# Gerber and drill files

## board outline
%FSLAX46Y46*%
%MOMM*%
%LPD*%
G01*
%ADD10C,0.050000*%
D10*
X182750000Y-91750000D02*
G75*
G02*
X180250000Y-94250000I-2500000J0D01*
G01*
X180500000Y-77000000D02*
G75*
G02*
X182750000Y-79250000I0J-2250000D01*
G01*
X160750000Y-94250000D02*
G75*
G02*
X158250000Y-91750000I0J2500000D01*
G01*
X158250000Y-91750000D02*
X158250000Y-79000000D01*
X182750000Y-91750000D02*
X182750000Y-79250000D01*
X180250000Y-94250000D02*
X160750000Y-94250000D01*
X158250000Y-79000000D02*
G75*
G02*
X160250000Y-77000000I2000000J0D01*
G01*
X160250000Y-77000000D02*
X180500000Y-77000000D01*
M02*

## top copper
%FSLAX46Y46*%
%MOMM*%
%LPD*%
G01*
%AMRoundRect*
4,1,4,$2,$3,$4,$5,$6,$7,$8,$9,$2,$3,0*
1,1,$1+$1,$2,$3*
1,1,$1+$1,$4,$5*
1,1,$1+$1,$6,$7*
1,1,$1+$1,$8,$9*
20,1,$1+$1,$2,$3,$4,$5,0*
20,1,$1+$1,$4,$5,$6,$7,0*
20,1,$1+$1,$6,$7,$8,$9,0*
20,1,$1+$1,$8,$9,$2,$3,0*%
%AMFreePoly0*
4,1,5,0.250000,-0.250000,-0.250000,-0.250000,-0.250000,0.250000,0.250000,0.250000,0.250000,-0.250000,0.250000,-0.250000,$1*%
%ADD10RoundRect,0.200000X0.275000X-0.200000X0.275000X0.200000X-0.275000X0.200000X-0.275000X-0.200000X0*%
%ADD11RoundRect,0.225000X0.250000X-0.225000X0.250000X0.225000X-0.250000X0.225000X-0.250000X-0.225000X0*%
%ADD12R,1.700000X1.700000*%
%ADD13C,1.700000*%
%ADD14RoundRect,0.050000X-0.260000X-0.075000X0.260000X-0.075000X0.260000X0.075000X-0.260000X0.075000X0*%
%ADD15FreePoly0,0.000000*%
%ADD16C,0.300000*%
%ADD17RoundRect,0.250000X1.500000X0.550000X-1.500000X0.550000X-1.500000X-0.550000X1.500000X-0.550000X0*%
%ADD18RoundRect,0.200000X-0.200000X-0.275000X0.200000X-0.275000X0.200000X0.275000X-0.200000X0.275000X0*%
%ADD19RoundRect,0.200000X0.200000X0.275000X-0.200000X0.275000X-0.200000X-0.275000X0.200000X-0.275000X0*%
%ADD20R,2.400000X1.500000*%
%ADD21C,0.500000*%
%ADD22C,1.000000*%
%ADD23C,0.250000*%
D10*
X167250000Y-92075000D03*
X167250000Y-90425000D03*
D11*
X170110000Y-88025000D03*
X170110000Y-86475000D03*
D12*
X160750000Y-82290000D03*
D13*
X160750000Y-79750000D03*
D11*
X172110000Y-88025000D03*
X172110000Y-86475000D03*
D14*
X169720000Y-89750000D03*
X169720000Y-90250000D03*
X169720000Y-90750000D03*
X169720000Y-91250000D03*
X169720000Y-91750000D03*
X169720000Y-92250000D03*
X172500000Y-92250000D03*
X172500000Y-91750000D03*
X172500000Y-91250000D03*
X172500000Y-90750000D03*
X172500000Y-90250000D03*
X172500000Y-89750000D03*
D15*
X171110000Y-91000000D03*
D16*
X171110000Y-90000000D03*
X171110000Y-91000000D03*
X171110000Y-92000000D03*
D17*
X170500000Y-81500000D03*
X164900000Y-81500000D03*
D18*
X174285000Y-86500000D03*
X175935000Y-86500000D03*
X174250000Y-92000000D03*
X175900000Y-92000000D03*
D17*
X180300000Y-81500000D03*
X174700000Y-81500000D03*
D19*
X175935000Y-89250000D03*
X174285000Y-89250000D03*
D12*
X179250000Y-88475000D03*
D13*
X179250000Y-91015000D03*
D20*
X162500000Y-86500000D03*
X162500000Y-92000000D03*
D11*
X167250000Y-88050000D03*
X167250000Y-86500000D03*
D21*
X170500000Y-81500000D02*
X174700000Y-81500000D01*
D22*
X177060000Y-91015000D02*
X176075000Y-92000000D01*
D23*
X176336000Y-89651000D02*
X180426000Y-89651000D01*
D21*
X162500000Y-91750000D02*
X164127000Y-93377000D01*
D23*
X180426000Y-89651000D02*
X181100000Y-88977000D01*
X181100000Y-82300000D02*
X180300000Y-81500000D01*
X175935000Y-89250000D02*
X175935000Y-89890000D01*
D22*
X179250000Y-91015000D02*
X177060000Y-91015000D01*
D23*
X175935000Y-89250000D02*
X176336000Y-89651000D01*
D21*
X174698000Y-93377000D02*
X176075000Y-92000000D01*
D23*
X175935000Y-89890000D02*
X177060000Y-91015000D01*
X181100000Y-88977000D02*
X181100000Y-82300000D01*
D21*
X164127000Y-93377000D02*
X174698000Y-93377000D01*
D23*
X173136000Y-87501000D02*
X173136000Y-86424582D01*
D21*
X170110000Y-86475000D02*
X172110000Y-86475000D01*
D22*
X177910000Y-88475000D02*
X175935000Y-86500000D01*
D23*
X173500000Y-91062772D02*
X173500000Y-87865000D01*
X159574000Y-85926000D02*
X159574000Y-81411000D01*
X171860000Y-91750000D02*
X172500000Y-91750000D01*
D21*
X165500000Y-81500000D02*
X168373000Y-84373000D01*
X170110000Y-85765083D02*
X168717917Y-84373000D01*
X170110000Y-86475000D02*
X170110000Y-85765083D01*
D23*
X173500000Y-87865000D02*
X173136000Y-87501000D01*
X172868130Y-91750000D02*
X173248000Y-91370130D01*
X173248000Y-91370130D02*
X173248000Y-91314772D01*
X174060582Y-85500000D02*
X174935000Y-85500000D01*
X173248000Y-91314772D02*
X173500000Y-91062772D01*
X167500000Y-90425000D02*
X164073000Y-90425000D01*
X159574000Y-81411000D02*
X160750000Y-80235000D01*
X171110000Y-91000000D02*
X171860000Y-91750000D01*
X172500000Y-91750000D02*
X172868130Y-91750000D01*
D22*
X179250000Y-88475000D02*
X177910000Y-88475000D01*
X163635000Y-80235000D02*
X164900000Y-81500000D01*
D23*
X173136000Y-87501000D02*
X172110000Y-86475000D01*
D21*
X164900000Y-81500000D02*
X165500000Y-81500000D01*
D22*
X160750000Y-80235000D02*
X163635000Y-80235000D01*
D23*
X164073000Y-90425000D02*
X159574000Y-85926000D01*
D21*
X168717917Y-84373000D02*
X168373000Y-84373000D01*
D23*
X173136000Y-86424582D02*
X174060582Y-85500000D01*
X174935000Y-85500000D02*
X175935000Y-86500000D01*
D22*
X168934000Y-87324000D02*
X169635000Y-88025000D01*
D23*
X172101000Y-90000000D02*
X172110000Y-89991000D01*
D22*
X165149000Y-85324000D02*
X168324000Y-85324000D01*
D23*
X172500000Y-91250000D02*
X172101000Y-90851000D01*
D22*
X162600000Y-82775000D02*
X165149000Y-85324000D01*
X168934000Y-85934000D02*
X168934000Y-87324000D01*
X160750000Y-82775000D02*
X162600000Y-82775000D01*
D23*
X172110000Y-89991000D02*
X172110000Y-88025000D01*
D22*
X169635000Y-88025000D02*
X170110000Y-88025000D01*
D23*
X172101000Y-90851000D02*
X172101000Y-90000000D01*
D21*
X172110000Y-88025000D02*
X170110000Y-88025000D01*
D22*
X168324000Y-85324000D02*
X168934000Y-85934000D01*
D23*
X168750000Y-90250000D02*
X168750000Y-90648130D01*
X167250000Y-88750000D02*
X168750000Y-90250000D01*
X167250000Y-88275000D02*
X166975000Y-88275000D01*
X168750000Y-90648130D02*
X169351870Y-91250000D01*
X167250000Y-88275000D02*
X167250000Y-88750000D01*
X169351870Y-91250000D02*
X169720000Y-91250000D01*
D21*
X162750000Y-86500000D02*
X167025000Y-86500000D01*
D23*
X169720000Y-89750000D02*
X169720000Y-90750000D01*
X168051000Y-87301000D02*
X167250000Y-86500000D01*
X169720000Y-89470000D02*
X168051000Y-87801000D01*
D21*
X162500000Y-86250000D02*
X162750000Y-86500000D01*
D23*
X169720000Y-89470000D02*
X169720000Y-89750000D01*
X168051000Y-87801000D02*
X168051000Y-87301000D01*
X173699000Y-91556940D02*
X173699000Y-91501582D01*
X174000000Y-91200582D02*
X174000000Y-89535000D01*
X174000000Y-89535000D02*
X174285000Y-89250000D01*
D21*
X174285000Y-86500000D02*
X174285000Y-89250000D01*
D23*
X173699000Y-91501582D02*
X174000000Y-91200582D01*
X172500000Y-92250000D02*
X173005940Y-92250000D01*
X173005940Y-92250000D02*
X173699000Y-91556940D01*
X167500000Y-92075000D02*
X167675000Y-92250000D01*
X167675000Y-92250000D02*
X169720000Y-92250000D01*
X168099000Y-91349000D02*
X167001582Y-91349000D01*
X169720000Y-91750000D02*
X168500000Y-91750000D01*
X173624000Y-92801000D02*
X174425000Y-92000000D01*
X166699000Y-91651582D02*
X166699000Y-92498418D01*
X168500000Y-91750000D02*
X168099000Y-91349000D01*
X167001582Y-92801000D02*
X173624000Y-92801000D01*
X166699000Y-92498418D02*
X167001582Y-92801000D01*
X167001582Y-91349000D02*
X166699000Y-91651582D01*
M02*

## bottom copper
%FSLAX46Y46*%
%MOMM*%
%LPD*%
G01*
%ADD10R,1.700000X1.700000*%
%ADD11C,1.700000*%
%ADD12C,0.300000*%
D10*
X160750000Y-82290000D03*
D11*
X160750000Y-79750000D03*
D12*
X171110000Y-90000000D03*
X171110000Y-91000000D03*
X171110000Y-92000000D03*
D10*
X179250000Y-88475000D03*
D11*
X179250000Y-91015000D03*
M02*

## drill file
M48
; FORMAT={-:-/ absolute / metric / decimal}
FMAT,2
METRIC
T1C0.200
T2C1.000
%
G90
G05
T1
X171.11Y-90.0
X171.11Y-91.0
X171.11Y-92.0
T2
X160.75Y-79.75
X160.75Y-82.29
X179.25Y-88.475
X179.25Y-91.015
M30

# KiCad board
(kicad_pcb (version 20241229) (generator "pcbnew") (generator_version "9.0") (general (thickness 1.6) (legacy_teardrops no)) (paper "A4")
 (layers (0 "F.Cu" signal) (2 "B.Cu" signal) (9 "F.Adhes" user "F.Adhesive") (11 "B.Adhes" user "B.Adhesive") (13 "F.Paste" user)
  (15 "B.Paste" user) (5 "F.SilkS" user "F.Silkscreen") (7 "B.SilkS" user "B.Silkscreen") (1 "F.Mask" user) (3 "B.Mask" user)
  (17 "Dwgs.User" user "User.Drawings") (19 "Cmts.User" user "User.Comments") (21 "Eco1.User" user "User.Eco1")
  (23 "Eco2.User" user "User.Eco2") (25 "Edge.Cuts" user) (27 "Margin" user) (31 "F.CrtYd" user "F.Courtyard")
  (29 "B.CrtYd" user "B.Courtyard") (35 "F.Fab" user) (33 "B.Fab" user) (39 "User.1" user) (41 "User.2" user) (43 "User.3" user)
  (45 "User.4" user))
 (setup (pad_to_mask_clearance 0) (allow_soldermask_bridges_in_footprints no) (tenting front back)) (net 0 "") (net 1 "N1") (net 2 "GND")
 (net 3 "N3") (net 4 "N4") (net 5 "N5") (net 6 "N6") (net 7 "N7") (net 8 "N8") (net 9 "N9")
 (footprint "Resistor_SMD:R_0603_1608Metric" (layer "F.Cu") (at 167.25 91.25 90)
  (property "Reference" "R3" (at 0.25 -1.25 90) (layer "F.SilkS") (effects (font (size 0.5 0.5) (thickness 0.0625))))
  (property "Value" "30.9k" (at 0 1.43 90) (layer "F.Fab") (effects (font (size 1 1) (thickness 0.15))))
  (pad "1" smd roundrect (at -0.825 0 90) (size 0.8 0.95) (layers "F.Cu" "F.Mask" "F.Paste") (roundrect_rratio 0.25) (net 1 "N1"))
  (pad "2" smd roundrect (at 0.825 0 90) (size 0.8 0.95) (layers "F.Cu" "F.Mask" "F.Paste") (roundrect_rratio 0.25) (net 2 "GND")))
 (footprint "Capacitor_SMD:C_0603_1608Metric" (layer "F.Cu") (at 170.11 87.25 90)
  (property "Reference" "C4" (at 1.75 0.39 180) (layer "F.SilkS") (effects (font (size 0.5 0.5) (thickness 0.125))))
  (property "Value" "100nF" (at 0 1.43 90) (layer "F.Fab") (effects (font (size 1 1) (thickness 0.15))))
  (pad "1" smd roundrect (at -0.775 0 90) (size 0.9 0.95) (layers "F.Cu" "F.Mask" "F.Paste") (roundrect_rratio 0.25) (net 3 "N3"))
  (pad "2" smd roundrect (at 0.775 0 90) (size 0.9 0.95) (layers "F.Cu" "F.Mask" "F.Paste") (roundrect_rratio 0.25) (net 2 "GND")))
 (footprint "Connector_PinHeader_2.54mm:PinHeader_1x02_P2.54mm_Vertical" (layer "F.Cu") (at 160.75 82.29 180)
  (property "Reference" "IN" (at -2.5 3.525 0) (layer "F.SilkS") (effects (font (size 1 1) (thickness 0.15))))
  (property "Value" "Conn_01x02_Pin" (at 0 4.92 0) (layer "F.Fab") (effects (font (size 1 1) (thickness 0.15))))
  (pad "1" thru_hole rect (at 0 0 180) (size 1.7 1.7) (drill 1) (layers "*.Cu" "*.Mask") (remove_unused_layers no) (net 3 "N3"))
  (pad "2" thru_hole circle (at 0 2.54 180) (size 1.7 1.7) (drill 1) (layers "*.Cu" "*.Mask") (remove_unused_layers no) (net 2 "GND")))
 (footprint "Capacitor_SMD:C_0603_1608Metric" (layer "F.Cu") (at 172.11 87.25 90)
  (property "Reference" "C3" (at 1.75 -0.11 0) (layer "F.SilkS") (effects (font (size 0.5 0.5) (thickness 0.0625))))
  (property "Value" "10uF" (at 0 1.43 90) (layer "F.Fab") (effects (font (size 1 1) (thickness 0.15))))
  (pad "1" smd roundrect (at -0.775 0 90) (size 0.9 0.95) (layers "F.Cu" "F.Mask" "F.Paste") (roundrect_rratio 0.25) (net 3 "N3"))
  (pad "2" smd roundrect (at 0.775 0 90) (size 0.9 0.95) (layers "F.Cu" "F.Mask" "F.Paste") (roundrect_rratio 0.25) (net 2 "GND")))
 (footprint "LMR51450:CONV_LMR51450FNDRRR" (layer "F.Cu") (at 171.11 91)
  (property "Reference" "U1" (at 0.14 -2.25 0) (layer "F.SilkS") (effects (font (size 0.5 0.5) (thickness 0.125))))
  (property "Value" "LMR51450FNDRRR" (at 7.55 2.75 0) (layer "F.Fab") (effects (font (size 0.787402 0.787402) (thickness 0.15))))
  (pad "1" smd roundrect (at -1.39 -1.25) (size 0.62 0.25) (layers "F.Cu" "F.Paste") (roundrect_rratio 0.2) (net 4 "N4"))
  (pad "2" smd roundrect (at -1.39 -0.75) (size 0.62 0.25) (layers "F.Cu" "F.Paste") (roundrect_rratio 0.2) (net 4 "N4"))
  (pad "3" smd roundrect (at -1.39 -0.25) (size 0.62 0.25) (layers "F.Cu" "F.Paste") (roundrect_rratio 0.2) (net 4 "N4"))
  (pad "4" smd roundrect (at -1.39 0.25) (size 0.62 0.25) (layers "F.Cu" "F.Paste") (roundrect_rratio 0.2) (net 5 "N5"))
  (pad "5" smd roundrect (at -1.39 0.75) (size 0.62 0.25) (layers "F.Cu" "F.Paste") (roundrect_rratio 0.2) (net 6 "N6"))
  (pad "6" smd roundrect (at -1.39 1.25) (size 0.62 0.25) (layers "F.Cu" "F.Paste") (roundrect_rratio 0.2) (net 1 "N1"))
  (pad "7" smd roundrect (at 1.39 1.25) (size 0.62 0.25) (layers "F.Cu" "F.Paste") (roundrect_rratio 0.2) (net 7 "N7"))
  (pad "8" smd roundrect (at 1.39 0.75) (size 0.62 0.25) (layers "F.Cu" "F.Paste") (roundrect_rratio 0.2) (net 2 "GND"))
  (pad "9" smd roundrect (at 1.39 0.25) (size 0.62 0.25) (layers "F.Cu" "F.Paste") (roundrect_rratio 0.2) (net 3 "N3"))
  (pad "10" smd roundrect (at 1.39 -0.25) (size 0.62 0.25) (layers "F.Cu" "F.Paste") (roundrect_rratio 0.2) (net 3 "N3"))
  (pad "11" smd roundrect (at 1.39 -0.75) (size 0.62 0.25) (layers "F.Cu" "F.Paste") (roundrect_rratio 0.2) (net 3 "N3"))
  (pad "12" smd roundrect (at 1.39 -1.25) (size 0.62 0.25) (layers "F.Cu" "F.Paste") (roundrect_rratio 0.2) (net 3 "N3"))
  (pad "13" smd custom (at 0 0) (size 0.5 0.5) (layers "F.Cu") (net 2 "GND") (options (clearance outline) (anchor rect)) (primitives))
  (pad "14" thru_hole circle (at 0 -1) (size 0.3 0.3) (drill 0.2) (layers "*.Cu") (remove_unused_layers no))
  (pad "15" thru_hole circle (at 0 0) (size 0.3 0.3) (drill 0.2) (layers "*.Cu") (remove_unused_layers no) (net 2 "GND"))
  (pad "16" thru_hole circle (at 0 1) (size 0.3 0.3) (drill 0.2) (layers "*.Cu") (remove_unused_layers no)))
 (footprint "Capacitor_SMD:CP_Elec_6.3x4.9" (layer "F.Cu") (at 167.7 81.5 180)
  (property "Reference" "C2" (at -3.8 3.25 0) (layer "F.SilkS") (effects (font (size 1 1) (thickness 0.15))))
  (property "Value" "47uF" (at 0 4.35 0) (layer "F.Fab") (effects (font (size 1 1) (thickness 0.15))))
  (pad "1" smd roundrect (at -2.8 0 180) (size 3.5 1.6) (layers "F.Cu" "F.Mask" "F.Paste") (roundrect_rratio 0.15625) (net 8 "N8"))
  (pad "2" smd roundrect (at 2.8 0 180) (size 3.5 1.6) (layers "F.Cu" "F.Mask" "F.Paste") (roundrect_rratio 0.15625) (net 2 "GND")))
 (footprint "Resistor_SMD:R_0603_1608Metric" (layer "F.Cu") (at 175.11 86.5)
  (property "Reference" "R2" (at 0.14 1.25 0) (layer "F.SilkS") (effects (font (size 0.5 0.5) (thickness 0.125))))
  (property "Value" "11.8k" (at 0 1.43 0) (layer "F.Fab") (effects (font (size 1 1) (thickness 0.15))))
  (pad "1" smd roundrect (at -0.825 0) (size 0.8 0.95) (layers "F.Cu" "F.Mask" "F.Paste") (roundrect_rratio 0.25) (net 7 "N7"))
  (pad "2" smd roundrect (at 0.825 0) (size 0.8 0.95) (layers "F.Cu" "F.Mask" "F.Paste") (roundrect_rratio 0.25) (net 2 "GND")))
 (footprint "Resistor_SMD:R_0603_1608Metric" (layer "F.Cu") (at 175.075 92)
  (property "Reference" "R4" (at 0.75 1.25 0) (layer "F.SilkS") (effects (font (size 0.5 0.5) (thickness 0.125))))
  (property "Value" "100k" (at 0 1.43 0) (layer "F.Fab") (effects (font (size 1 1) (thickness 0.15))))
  (pad "1" smd roundrect (at -0.825 0) (size 0.8 0.95) (layers "F.Cu" "F.Mask" "F.Paste") (roundrect_rratio 0.25) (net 6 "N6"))
  (pad "2" smd roundrect (at 0.825 0) (size 0.8 0.95) (layers "F.Cu" "F.Mask" "F.Paste") (roundrect_rratio 0.25) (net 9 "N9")))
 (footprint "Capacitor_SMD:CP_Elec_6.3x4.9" (layer "F.Cu") (at 177.5 81.5 180)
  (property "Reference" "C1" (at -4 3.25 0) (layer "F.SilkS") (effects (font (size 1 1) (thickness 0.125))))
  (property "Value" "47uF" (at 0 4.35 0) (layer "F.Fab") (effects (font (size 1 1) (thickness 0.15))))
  (pad "1" smd roundrect (at -2.8 0 180) (size 3.5 1.6) (layers "F.Cu" "F.Mask" "F.Paste") (roundrect_rratio 0.15625) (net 9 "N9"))
  (pad "2" smd roundrect (at 2.8 0 180) (size 3.5 1.6) (layers "F.Cu" "F.Mask" "F.Paste") (roundrect_rratio 0.15625) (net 8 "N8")))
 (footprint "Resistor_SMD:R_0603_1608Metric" (layer "F.Cu") (at 175.11 89.25 180)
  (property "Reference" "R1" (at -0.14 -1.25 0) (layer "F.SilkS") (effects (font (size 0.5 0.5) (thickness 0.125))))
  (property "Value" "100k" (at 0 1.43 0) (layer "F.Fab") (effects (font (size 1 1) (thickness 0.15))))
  (pad "1" smd roundrect (at -0.825 0 180) (size 0.8 0.95) (layers "F.Cu" "F.Mask" "F.Paste") (roundrect_rratio 0.25) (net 9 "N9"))
  (pad "2" smd roundrect (at 0.825 0 180) (size 0.8 0.95) (layers "F.Cu" "F.Mask" "F.Paste") (roundrect_rratio 0.25) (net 7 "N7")))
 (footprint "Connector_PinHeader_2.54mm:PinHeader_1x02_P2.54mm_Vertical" (layer "F.Cu") (at 179.25 88.475)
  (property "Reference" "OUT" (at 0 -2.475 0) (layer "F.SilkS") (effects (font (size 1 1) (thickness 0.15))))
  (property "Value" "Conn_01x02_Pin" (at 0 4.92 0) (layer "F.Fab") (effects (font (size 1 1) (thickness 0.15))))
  (pad "1" thru_hole rect (at 0 0) (size 1.7 1.7) (drill 1) (layers "*.Cu" "*.Mask") (remove_unused_layers no) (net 2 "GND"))
  (pad "2" thru_hole circle (at 0 2.54) (size 1.7 1.7) (drill 1) (layers "*.Cu" "*.Mask") (remove_unused_layers no) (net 9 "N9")))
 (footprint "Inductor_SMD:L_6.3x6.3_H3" (layer "F.Cu") (at 162.5 89.25 -90)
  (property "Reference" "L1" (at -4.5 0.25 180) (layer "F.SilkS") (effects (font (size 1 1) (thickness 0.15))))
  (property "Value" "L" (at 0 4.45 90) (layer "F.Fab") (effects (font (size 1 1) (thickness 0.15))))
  (pad "1" smd rect (at -2.75 0 270) (size 1.5 2.4) (layers "F.Cu" "F.Mask" "F.Paste") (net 4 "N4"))
  (pad "2" smd rect (at 2.75 0 270) (size 1.5 2.4) (layers "F.Cu" "F.Mask" "F.Paste") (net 9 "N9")))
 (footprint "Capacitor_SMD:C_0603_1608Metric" (layer "F.Cu") (at 167.25 87.275 90)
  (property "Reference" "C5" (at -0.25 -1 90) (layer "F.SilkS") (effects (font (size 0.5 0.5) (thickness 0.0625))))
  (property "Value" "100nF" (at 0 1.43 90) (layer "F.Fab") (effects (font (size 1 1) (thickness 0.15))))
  (pad "1" smd roundrect (at -0.775 0 90) (size 0.9 0.95) (layers "F.Cu" "F.Mask" "F.Paste") (roundrect_rratio 0.25) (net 5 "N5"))
  (pad "2" smd roundrect (at 0.775 0 90) (size 0.9 0.95) (layers "F.Cu" "F.Mask" "F.Paste") (roundrect_rratio 0.25) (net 4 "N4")))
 (gr_arc (start 182.75 91.75) (mid 182.017767 93.517767) (end 180.25 94.25) (stroke (width 0.05) (type default)) (layer "Edge.Cuts"))
 (gr_arc (start 180.5 77) (mid 182.09099 77.65901) (end 182.75 79.25) (stroke (width 0.05) (type default)) (layer "Edge.Cuts"))
 (gr_arc (start 160.75 94.25) (mid 158.982233 93.517767) (end 158.25 91.75) (stroke (width 0.05) (type default)) (layer "Edge.Cuts"))
 (gr_line (start 158.25 91.75) (end 158.25 79) (stroke (width 0.05) (type default)) (layer "Edge.Cuts"))
 (gr_line (start 182.75 91.75) (end 182.75 79.25) (stroke (width 0.05) (type default)) (layer "Edge.Cuts"))
 (gr_line (start 180.25 94.25) (end 160.75 94.25) (stroke (width 0.05) (type default)) (layer "Edge.Cuts"))
 (gr_arc (start 158.25 79) (mid 158.835786 77.585786) (end 160.25 77) (stroke (width 0.05) (type default)) (layer "Edge.Cuts"))
 (gr_line (start 160.25 77) (end 180.5 77) (stroke (width 0.05) (type default)) (layer "Edge.Cuts"))
 (segment (start 170.5 81.5) (end 174.7 81.5) (width 0.5) (layer "F.Cu") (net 8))
 (segment (start 177.06 91.015) (end 176.075 92) (width 1) (layer "F.Cu") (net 9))
 (segment (start 176.336 89.651) (end 180.426 89.651) (width 0.25) (layer "F.Cu") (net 9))
 (segment (start 162.5 91.75) (end 164.127 93.377) (width 0.5) (layer "F.Cu") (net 9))
 (segment (start 180.426 89.651) (end 181.1 88.977) (width 0.25) (layer "F.Cu") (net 9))
 (segment (start 181.1 82.3) (end 180.3 81.5) (width 0.25) (layer "F.Cu") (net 9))
 (segment (start 175.935 89.25) (end 175.935 89.89) (width 0.25) (layer "F.Cu") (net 9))
 (segment (start 179.25 91.015) (end 177.06 91.015) (width 1) (layer "F.Cu") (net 9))
 (segment (start 175.935 89.25) (end 176.336 89.651) (width 0.25) (layer "F.Cu") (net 9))
 (segment (start 174.698 93.377) (end 176.075 92) (width 0.5) (layer "F.Cu") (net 9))
 (segment (start 175.935 89.89) (end 177.06 91.015) (width 0.25) (layer "F.Cu") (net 9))
 (segment (start 181.1 88.977) (end 181.1 82.3) (width 0.25) (layer "F.Cu") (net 9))
 (segment (start 164.127 93.377) (end 174.698 93.377) (width 0.5) (layer "F.Cu") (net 9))
 (segment (start 173.136 87.501) (end 173.136 86.424582) (width 0.25) (layer "F.Cu") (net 2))
 (segment (start 170.11 86.475) (end 172.11 86.475) (width 0.5) (layer "F.Cu") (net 2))
 (segment (start 177.91 88.475) (end 175.935 86.5) (width 1) (layer "F.Cu") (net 2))
 (segment (start 173.5 91.062772) (end 173.5 87.865) (width 0.25) (layer "F.Cu") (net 2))
 (segment (start 159.574 85.926) (end 159.574 81.411) (width 0.25) (layer "F.Cu") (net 2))
 (segment (start 171.86 91.75) (end 172.5 91.75) (width 0.25) (layer "F.Cu") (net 2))
 (segment (start 165.5 81.5) (end 168.373 84.373) (width 0.5) (layer "F.Cu") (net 2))
 (segment (start 170.11 85.765083) (end 168.717917 84.373) (width 0.5) (layer "F.Cu") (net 2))
 (segment (start 170.11 86.475) (end 170.11 85.765083) (width 0.5) (layer "F.Cu") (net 2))
 (segment (start 173.5 87.865) (end 173.136 87.501) (width 0.25) (layer "F.Cu") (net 2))
 (segment (start 172.86813 91.75) (end 173.248 91.37013) (width 0.25) (layer "F.Cu") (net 2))
 (segment (start 173.248 91.37013) (end 173.248 91.314772) (width 0.25) (layer "F.Cu") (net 2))
 (segment (start 174.060582 85.5) (end 174.935 85.5) (width 0.25) (layer "F.Cu") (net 2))
 (segment (start 173.248 91.314772) (end 173.5 91.062772) (width 0.25) (layer "F.Cu") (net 2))
 (segment (start 167.5 90.425) (end 164.073 90.425) (width 0.25) (layer "F.Cu") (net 2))
 (segment (start 159.574 81.411) (end 160.75 80.235) (width 0.25) (layer "F.Cu") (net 2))
 (segment (start 171.11 91) (end 171.86 91.75) (width 0.25) (layer "F.Cu") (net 2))
 (segment (start 172.5 91.75) (end 172.86813 91.75) (width 0.25) (layer "F.Cu") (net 2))
 (segment (start 179.25 88.475) (end 177.91 88.475) (width 1) (layer "F.Cu") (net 2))
 (segment (start 163.635 80.235) (end 164.9 81.5) (width 1) (layer "F.Cu") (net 2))
 (segment (start 173.136 87.501) (end 172.11 86.475) (width 0.25) (layer "F.Cu") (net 2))
 (segment (start 164.9 81.5) (end 165.5 81.5) (width 0.5) (layer "F.Cu") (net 2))
 (segment (start 160.75 80.235) (end 163.635 80.235) (width 1) (layer "F.Cu") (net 2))
 (segment (start 164.073 90.425) (end 159.574 85.926) (width 0.25) (layer "F.Cu") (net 2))
 (segment (start 168.717917 84.373) (end 168.373 84.373) (width 0.5) (layer "F.Cu") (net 2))
 (segment (start 173.136 86.424582) (end 174.060582 85.5) (width 0.25) (layer "F.Cu") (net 2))
 (segment (start 174.935 85.5) (end 175.935 86.5) (width 0.25) (layer "F.Cu") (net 2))
 (segment (start 168.934 87.324) (end 169.635 88.025) (width 1) (layer "F.Cu") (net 3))
 (segment (start 172.101 90) (end 172.11 89.991) (width 0.25) (layer "F.Cu") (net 3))
 (segment (start 165.149 85.324) (end 168.324 85.324) (width 1) (layer "F.Cu") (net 3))
 (segment (start 172.5 91.25) (end 172.101 90.851) (width 0.25) (layer "F.Cu") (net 3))
 (segment (start 162.6 82.775) (end 165.149 85.324) (width 1) (layer "F.Cu") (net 3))
 (segment (start 168.934 85.934) (end 168.934 87.324) (width 1) (layer "F.Cu") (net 3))
 (segment (start 160.75 82.775) (end 162.6 82.775) (width 1) (layer "F.Cu") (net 3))
 (segment (start 172.11 89.991) (end 172.11 88.025) (width 0.25) (layer "F.Cu") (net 3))
 (segment (start 169.635 88.025) (end 170.11 88.025) (width 1) (layer "F.Cu") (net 3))
 (segment (start 172.101 90.851) (end 172.101 90) (width 0.25) (layer "F.Cu") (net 3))
 (segment (start 172.11 88.025) (end 170.11 88.025) (width 0.5) (layer "F.Cu") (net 3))
 (segment (start 168.324 85.324) (end 168.934 85.934) (width 1) (layer "F.Cu") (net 3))
 (segment (start 168.75 90.25) (end 168.75 90.64813) (width 0.25) (layer "F.Cu") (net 5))
 (segment (start 167.25 88.75) (end 168.75 90.25) (width 0.25) (layer "F.Cu") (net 5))
 (segment (start 167.25 88.275) (end 166.975 88.275) (width 0.25) (layer "F.Cu") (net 5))
 (segment (start 168.75 90.64813) (end 169.35187 91.25) (width 0.25) (layer "F.Cu") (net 5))
 (segment (start 167.25 88.275) (end 167.25 88.75) (width 0.25) (layer "F.Cu") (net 5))
 (segment (start 169.35187 91.25) (end 169.72 91.25) (width 0.25) (layer "F.Cu") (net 5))
 (segment (start 162.75 86.5) (end 167.025 86.5) (width 0.5) (layer "F.Cu") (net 4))
 (segment (start 169.72 89.75) (end 169.72 90.75) (width 0.25) (layer "F.Cu") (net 4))
 (segment (start 168.051 87.301) (end 167.25 86.5) (width 0.25) (layer "F.Cu") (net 4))
 (segment (start 169.72 89.47) (end 168.051 87.801) (width 0.25) (layer "F.Cu") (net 4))
 (segment (start 162.5 86.25) (end 162.75 86.5) (width 0.5) (layer "F.Cu") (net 4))
 (segment (start 169.72 89.47) (end 169.72 89.75) (width 0.25) (layer "F.Cu") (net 4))
 (segment (start 168.051 87.801) (end 168.051 87.301) (width 0.25) (layer "F.Cu") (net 4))
 (segment (start 173.699 91.55694) (end 173.699 91.501582) (width 0.25) (layer "F.Cu") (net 7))
 (segment (start 174 91.200582) (end 174 89.535) (width 0.25) (layer "F.Cu") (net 7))
 (segment (start 174 89.535) (end 174.285 89.25) (width 0.25) (layer "F.Cu") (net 7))
 (segment (start 174.285 86.5) (end 174.285 89.25) (width 0.5) (layer "F.Cu") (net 7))
 (segment (start 173.699 91.501582) (end 174 91.200582) (width 0.25) (layer "F.Cu") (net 7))
 (segment (start 172.5 92.25) (end 173.00594 92.25) (width 0.25) (layer "F.Cu") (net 7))
 (segment (start 173.00594 92.25) (end 173.699 91.55694) (width 0.25) (layer "F.Cu") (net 7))
 (segment (start 167.5 92.075) (end 167.675 92.25) (width 0.25) (layer "F.Cu") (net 1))
 (segment (start 167.675 92.25) (end 169.72 92.25) (width 0.25) (layer "F.Cu") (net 1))
 (segment (start 168.099 91.349) (end 167.001582 91.349) (width 0.25) (layer "F.Cu") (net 6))
 (segment (start 169.72 91.75) (end 168.5 91.75) (width 0.25) (layer "F.Cu") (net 6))
 (segment (start 173.624 92.801) (end 174.425 92) (width 0.25) (layer "F.Cu") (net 6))
 (segment (start 166.699 91.651582) (end 166.699 92.498418) (width 0.25) (layer "F.Cu") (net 6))
 (segment (start 168.5 91.75) (end 168.099 91.349) (width 0.25) (layer "F.Cu") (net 6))
 (segment (start 167.001582 92.801) (end 173.624 92.801) (width 0.25) (layer "F.Cu") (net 6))
 (segment (start 166.699 92.498418) (end 167.001582 92.801) (width 0.25) (layer "F.Cu") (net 6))
 (segment (start 167.001582 91.349) (end 166.699 91.651582) (width 0.25) (layer "F.Cu") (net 6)))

